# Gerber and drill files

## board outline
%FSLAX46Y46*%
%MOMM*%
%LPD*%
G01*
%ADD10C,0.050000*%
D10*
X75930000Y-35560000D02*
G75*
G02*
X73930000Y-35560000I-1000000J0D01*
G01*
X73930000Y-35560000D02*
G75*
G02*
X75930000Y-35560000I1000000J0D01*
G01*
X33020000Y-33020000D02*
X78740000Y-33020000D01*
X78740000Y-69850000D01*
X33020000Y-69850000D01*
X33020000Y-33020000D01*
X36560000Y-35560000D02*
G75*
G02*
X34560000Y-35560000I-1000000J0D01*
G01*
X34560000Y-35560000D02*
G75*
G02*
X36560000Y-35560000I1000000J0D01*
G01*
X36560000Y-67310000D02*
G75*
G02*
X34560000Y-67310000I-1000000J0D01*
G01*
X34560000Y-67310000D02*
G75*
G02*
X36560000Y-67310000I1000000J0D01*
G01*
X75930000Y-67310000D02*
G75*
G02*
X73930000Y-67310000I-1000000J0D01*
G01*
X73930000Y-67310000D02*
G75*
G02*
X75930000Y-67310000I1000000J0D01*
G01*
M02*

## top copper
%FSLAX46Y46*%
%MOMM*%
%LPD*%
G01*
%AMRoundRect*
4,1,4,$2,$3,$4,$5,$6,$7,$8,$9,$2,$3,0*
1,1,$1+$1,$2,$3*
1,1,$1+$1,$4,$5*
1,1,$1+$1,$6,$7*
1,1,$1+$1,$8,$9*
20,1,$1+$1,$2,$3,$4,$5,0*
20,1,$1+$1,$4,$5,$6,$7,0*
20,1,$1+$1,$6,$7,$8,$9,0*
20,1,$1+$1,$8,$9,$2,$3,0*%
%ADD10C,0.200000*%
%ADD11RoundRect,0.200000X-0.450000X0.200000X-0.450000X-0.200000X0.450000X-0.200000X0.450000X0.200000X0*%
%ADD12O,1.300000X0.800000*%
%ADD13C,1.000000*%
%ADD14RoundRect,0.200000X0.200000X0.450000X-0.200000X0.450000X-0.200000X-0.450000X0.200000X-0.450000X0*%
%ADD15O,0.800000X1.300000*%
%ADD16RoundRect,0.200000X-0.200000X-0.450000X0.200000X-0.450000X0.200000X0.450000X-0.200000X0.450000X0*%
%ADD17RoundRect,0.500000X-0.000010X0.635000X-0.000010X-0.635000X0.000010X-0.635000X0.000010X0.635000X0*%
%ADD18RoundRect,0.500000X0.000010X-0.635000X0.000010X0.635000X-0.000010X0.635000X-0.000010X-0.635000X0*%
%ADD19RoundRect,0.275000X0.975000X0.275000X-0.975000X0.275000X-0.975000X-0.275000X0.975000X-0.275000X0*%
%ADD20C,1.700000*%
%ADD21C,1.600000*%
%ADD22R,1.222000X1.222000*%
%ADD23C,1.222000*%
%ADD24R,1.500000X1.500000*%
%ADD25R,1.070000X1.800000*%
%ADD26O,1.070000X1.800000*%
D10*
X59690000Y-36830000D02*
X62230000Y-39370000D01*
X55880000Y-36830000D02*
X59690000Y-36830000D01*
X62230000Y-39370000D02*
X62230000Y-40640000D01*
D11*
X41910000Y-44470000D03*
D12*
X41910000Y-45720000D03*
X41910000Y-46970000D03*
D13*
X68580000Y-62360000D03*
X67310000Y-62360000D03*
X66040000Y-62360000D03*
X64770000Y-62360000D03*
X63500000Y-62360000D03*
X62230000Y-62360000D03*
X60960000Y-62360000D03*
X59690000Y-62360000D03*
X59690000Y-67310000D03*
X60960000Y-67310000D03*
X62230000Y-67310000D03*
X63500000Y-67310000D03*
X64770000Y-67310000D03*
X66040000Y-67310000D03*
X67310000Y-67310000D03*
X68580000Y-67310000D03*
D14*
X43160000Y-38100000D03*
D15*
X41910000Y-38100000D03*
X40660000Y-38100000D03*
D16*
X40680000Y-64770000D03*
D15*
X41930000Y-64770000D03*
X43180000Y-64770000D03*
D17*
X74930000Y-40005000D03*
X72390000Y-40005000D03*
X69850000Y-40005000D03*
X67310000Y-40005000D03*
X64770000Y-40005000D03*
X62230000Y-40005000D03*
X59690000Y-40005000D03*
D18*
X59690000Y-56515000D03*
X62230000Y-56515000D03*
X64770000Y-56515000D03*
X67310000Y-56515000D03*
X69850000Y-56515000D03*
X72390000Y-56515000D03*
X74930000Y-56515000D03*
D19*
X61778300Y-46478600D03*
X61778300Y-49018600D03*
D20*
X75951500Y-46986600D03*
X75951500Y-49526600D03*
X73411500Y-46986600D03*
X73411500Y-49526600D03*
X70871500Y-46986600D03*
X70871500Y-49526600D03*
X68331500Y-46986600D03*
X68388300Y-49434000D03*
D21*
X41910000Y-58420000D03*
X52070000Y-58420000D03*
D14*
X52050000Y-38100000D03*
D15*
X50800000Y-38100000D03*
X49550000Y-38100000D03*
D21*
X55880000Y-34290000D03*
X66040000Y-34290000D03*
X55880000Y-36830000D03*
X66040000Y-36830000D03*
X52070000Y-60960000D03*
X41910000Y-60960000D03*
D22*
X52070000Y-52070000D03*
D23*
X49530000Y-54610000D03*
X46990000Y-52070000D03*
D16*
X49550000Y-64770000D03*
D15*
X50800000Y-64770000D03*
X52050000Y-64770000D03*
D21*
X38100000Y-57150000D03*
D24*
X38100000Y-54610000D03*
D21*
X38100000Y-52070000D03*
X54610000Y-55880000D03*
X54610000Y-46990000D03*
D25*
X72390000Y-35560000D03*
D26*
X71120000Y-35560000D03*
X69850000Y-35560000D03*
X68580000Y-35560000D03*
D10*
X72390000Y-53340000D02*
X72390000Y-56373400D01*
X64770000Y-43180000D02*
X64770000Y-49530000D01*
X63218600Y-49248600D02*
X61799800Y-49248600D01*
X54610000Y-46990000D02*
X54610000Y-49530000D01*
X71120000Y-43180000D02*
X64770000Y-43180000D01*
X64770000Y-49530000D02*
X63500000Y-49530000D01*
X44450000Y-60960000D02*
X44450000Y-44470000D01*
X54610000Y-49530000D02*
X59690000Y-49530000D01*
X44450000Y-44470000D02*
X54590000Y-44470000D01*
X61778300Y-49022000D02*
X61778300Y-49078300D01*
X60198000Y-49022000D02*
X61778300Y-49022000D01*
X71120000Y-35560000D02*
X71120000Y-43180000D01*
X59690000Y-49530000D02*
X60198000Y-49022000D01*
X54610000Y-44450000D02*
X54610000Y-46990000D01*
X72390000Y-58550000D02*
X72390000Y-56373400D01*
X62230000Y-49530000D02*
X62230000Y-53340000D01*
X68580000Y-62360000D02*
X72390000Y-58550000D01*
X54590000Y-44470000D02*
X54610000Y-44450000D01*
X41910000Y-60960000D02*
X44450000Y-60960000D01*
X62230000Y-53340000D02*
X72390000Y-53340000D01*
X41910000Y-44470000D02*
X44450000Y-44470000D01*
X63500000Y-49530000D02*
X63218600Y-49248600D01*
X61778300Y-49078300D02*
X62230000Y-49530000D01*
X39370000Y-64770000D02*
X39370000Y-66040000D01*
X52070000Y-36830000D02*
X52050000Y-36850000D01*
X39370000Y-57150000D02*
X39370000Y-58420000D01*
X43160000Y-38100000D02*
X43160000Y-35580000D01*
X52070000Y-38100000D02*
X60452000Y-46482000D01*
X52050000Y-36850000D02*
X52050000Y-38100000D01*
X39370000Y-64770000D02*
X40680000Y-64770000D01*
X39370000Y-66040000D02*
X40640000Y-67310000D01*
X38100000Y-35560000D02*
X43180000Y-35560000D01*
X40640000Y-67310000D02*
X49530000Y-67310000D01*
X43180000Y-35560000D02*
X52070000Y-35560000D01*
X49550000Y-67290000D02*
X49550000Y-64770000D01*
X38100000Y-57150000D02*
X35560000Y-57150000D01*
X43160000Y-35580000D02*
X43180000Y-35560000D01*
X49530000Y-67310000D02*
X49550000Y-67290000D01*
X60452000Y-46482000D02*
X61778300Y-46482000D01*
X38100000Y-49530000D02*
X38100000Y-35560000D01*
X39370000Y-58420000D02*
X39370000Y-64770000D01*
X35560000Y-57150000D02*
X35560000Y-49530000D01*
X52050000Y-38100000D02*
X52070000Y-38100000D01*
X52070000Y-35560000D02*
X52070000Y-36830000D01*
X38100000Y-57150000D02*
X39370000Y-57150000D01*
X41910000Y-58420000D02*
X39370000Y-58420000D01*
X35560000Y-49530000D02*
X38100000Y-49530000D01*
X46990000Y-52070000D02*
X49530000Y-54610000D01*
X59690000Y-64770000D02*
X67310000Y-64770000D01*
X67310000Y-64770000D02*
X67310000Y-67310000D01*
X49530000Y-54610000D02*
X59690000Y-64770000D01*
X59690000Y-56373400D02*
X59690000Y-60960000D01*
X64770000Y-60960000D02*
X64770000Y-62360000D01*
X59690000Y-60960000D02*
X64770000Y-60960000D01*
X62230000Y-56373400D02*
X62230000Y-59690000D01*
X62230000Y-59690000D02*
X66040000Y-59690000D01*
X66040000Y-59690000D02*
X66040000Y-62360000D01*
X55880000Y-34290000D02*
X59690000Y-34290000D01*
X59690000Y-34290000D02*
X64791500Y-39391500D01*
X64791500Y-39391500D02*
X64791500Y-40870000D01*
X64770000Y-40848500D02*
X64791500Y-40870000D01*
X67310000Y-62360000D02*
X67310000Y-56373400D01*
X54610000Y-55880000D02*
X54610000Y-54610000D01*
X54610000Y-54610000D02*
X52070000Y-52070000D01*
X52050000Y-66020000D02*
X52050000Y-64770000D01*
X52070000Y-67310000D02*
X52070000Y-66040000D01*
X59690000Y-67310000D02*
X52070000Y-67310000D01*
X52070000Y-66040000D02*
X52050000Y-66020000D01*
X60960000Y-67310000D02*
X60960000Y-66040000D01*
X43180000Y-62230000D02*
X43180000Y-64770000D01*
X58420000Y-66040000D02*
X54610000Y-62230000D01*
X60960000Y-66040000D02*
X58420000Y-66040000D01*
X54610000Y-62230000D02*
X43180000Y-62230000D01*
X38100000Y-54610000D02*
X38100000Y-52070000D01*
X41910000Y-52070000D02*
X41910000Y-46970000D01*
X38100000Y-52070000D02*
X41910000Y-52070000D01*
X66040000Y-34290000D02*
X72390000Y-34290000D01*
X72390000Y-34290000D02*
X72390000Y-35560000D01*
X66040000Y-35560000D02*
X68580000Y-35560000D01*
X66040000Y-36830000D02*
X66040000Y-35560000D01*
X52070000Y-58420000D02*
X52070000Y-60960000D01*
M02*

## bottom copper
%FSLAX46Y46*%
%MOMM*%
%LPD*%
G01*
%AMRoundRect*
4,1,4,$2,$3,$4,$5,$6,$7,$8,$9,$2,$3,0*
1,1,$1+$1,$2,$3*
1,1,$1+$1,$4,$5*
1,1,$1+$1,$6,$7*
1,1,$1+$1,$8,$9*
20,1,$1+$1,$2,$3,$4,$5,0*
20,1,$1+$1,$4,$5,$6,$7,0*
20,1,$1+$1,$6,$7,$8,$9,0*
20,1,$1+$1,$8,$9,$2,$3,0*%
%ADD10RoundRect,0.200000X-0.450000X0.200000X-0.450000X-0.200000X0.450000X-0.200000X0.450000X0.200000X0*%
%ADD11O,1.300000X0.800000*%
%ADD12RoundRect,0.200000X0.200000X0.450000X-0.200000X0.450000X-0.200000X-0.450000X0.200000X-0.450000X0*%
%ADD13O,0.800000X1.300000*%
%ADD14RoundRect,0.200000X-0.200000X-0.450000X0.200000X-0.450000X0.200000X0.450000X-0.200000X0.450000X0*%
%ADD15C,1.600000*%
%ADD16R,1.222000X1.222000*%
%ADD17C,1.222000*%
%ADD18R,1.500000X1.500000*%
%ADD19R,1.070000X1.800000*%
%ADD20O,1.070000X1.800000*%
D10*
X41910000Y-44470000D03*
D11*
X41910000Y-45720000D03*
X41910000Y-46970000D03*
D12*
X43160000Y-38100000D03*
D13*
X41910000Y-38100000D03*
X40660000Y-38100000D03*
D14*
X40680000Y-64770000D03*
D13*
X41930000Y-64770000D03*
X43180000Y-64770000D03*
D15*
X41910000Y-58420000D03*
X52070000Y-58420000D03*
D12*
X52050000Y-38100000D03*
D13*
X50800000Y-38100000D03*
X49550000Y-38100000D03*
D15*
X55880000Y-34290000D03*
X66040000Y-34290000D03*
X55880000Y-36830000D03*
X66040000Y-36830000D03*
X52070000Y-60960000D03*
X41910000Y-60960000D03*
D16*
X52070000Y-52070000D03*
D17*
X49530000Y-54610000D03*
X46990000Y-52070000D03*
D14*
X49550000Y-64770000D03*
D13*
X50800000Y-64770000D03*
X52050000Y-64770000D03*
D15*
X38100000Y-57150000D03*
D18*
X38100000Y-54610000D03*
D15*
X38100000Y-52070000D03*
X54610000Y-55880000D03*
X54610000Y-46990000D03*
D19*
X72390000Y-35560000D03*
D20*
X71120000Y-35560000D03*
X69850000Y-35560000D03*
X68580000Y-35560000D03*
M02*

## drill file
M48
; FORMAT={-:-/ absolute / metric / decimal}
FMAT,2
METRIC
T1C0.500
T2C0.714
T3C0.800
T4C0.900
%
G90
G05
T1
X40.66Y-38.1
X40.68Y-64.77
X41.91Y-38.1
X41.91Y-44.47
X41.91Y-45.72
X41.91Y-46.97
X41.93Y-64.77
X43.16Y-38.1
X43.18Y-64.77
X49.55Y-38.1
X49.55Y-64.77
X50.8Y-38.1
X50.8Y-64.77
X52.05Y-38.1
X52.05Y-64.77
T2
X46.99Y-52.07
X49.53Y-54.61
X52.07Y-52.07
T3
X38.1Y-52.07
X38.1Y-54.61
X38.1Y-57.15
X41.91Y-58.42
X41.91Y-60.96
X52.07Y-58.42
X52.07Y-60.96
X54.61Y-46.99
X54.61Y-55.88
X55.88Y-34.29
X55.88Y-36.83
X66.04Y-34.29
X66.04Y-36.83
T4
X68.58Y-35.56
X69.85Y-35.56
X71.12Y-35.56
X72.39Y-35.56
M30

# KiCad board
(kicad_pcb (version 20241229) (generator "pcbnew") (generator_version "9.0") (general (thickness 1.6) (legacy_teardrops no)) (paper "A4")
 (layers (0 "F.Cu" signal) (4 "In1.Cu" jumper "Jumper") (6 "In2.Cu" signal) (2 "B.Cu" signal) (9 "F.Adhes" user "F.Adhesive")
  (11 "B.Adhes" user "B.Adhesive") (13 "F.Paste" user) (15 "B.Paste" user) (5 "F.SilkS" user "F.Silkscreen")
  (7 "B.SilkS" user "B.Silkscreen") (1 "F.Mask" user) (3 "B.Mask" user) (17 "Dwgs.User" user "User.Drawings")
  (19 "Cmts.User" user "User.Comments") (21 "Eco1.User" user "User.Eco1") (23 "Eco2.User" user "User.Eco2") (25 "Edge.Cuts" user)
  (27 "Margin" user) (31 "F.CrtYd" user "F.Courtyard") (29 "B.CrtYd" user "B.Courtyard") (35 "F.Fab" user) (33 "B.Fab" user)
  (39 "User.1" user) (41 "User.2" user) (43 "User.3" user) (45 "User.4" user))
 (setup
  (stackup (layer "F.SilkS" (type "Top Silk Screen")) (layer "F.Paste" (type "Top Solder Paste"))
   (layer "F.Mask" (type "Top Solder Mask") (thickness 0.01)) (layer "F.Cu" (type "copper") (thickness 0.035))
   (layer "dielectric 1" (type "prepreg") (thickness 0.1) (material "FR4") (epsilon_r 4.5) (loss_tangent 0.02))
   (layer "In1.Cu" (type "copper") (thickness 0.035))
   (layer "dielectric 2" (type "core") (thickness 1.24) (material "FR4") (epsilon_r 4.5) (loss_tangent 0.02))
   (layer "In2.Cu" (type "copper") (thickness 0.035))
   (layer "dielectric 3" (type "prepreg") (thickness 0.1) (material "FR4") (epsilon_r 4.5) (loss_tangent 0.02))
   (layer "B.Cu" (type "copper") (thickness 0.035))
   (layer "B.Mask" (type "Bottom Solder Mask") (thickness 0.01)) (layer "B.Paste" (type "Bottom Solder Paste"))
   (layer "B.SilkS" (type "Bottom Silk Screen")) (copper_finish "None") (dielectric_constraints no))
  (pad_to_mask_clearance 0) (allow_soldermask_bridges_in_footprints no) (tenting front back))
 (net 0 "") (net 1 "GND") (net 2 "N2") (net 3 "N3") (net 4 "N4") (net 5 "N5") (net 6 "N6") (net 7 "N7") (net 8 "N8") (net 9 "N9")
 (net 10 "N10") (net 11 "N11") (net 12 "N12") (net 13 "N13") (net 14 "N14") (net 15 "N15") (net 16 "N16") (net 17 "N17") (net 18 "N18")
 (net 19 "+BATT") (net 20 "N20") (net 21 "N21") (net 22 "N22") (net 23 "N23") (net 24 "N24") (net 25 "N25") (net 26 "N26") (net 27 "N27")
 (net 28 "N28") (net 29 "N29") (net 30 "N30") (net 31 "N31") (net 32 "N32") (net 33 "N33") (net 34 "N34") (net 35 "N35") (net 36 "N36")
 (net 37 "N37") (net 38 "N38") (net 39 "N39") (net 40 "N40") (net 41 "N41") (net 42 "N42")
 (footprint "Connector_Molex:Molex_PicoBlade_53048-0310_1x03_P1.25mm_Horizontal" (layer "F.Cu") (at 41.91 44.47 -90)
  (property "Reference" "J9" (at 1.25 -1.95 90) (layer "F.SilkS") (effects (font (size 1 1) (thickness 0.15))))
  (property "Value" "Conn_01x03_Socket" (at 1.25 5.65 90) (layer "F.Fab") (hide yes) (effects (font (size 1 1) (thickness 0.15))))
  (pad "1" thru_hole roundrect (at 0 0 270) (size 0.8 1.3) (drill 0.5) (layers "*.Cu" "*.Mask") (remove_unused_layers no)
   (roundrect_rratio 0.25) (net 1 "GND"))
  (pad "2" thru_hole oval (at 1.25 0 270) (size 0.8 1.3) (drill 0.5) (layers "*.Cu" "*.Mask") (remove_unused_layers no) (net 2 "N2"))
  (pad "3" thru_hole oval (at 2.5 0 270) (size 0.8 1.3) (drill 0.5) (layers "*.Cu" "*.Mask") (remove_unused_layers no) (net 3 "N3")))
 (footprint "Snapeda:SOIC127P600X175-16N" (layer "F.Cu") (at 63.5 64.835 -90)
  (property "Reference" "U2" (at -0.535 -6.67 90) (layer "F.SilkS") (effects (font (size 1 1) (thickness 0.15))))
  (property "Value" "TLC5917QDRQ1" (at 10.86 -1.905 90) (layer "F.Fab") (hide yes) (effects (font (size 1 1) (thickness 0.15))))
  (pad "1" smd circle (at -2.475 -5.08 270) (size 1 1) (layers "F.Cu" "F.Mask" "F.Paste") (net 1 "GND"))
  (pad "2" smd circle (at -2.475 -3.81 270) (size 1 1) (layers "F.Cu" "F.Mask" "F.Paste") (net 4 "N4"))
  (pad "3" smd circle (at -2.475 -2.54 270) (size 1 1) (layers "F.Cu" "F.Mask" "F.Paste") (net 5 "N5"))
  (pad "4" smd circle (at -2.475 -1.27 270) (size 1 1) (layers "F.Cu" "F.Mask" "F.Paste") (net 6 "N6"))
  (pad "5" smd circle (at -2.475 0 270) (size 1 1) (layers "F.Cu" "F.Mask" "F.Paste") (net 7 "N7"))
  (pad "6" smd circle (at -2.475 1.27 270) (size 1 1) (layers "F.Cu" "F.Mask" "F.Paste") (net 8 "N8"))
  (pad "7" smd circle (at -2.475 2.54 270) (size 1 1) (layers "F.Cu" "F.Mask" "F.Paste") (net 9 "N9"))
  (pad "8" smd circle (at -2.475 3.81 270) (size 1 1) (layers "F.Cu" "F.Mask" "F.Paste") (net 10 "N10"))
  (pad "9" smd circle (at 2.475 3.81 270) (size 1 1) (layers "F.Cu" "F.Mask" "F.Paste") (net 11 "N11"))
  (pad "10" smd circle (at 2.475 2.54 270) (size 1 1) (layers "F.Cu" "F.Mask" "F.Paste") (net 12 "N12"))
  (pad "11" smd circle (at 2.475 1.27 270) (size 1 1) (layers "F.Cu" "F.Mask" "F.Paste") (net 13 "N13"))
  (pad "12" smd circle (at 2.475 0 270) (size 1 1) (layers "F.Cu" "F.Mask" "F.Paste") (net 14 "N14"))
  (pad "13" smd circle (at 2.475 -1.27 270) (size 1 1) (layers "F.Cu" "F.Mask" "F.Paste") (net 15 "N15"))
  (pad "14" smd circle (at 2.475 -2.54 270) (size 1 1) (layers "F.Cu" "F.Mask" "F.Paste") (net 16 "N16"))
  (pad "15" smd circle (at 2.475 -3.81 270) (size 1 1) (layers "F.Cu" "F.Mask" "F.Paste") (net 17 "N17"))
  (pad "16" smd circle (at 2.475 -5.08 270) (size 1 1) (layers "F.Cu" "F.Mask" "F.Paste") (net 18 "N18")))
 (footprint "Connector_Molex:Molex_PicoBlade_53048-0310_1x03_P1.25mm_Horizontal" (layer "F.Cu") (at 43.16 38.1 180)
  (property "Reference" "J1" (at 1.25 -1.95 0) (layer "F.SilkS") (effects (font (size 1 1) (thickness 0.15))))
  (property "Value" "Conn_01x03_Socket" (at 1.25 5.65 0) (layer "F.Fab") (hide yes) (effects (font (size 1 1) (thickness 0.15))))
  (pad "1" thru_hole roundrect (at 0 0 180) (size 0.8 1.3) (drill 0.5) (layers "*.Cu" "*.Mask") (remove_unused_layers no)
   (roundrect_rratio 0.25) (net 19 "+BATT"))
  (pad "2" thru_hole oval (at 1.25 0 180) (size 0.8 1.3) (drill 0.5) (layers "*.Cu" "*.Mask") (remove_unused_layers no) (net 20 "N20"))
  (pad "3" thru_hole oval (at 2.5 0 180) (size 0.8 1.3) (drill 0.5) (layers "*.Cu" "*.Mask") (remove_unused_layers no) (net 13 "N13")))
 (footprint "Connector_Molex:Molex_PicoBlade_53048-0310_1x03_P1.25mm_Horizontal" (layer "F.Cu") (at 40.68 64.77)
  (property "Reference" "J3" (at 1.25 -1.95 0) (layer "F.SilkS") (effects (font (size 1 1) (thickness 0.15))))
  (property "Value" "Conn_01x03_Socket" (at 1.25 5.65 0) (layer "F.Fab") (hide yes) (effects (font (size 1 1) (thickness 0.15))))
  (pad "1" thru_hole roundrect (at 0 0) (size 0.8 1.3) (drill 0.5) (layers "*.Cu" "*.Mask") (remove_unused_layers no)
   (roundrect_rratio 0.25) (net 19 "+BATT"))
  (pad "2" thru_hole oval (at 1.25 0) (size 0.8 1.3) (drill 0.5) (layers "*.Cu" "*.Mask") (remove_unused_layers no) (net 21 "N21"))
  (pad "3" thru_hole oval (at 2.5 0) (size 0.8 1.3) (drill 0.5) (layers "*.Cu" "*.Mask") (remove_unused_layers no) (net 12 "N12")))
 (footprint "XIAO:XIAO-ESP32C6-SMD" (layer "F.Cu") (at 67.31 48.26 -90)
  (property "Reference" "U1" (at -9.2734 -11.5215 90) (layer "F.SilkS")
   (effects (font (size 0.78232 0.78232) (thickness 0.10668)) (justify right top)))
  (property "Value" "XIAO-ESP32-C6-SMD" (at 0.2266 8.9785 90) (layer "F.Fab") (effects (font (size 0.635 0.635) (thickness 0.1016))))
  (pad "1" smd roundrect (at -7.62 -7.62 270) (size 2.27 1) (drill (offset -0.635 0)) (layers "F.Cu" "F.Mask" "F.Paste")
   (roundrect_rratio 0.5) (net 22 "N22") (solder_mask_margin 0.0508) (thermal_bridge_angle 45))
  (pad "2" smd roundrect (at -7.62 -5.08 270) (size 2.27 1) (drill (offset -0.635 0)) (layers "F.Cu" "F.Mask" "F.Paste")
   (roundrect_rratio 0.5) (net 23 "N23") (solder_mask_margin 0.0508) (thermal_bridge_angle 45))
  (pad "3" smd roundrect (at -7.62 -2.54 270) (size 2.27 1) (drill (offset -0.635 0)) (layers "F.Cu" "F.Mask" "F.Paste")
   (roundrect_rratio 0.5) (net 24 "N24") (solder_mask_margin 0.0508) (thermal_bridge_angle 45))
  (pad "4" smd roundrect (at -7.62 0 270) (size 2.27 1) (drill (offset -0.635 0)) (layers "F.Cu" "F.Mask" "F.Paste") (roundrect_rratio 0.5)
   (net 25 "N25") (solder_mask_margin 0.0508) (thermal_bridge_angle 45))
  (pad "5" smd roundrect (at -7.62 2.54 270) (size 2.27 1) (drill (offset -0.635 0)) (layers "F.Cu" "F.Mask" "F.Paste")
   (roundrect_rratio 0.5) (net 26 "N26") (solder_mask_margin 0.0508) (thermal_bridge_angle 45))
  (pad "6" smd roundrect (at -7.62 5.08 270) (size 2.27 1) (drill (offset -0.635 0)) (layers "F.Cu" "F.Mask" "F.Paste")
   (roundrect_rratio 0.5) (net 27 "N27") (solder_mask_margin 0.0508) (thermal_bridge_angle 45))
  (pad "7" smd roundrect (at -7.62 7.62 270) (size 2.27 1) (drill (offset -0.635 0)) (layers "F.Cu" "F.Mask" "F.Paste")
   (roundrect_rratio 0.5) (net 15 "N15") (solder_mask_margin 0.0508) (thermal_bridge_angle 45))
  (pad "8" smd roundrect (at 7.62 7.62 90) (size 2.27 1) (drill (offset -0.635 0)) (layers "F.Cu" "F.Mask" "F.Paste") (roundrect_rratio 0.5)
   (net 6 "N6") (solder_mask_margin 0.0508) (thermal_bridge_angle 45))
  (pad "9" smd roundrect (at 7.62 5.08 90) (size 2.27 1) (drill (offset -0.635 0)) (layers "F.Cu" "F.Mask" "F.Paste") (roundrect_rratio 0.5)
   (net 5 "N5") (solder_mask_margin 0.0508) (thermal_bridge_angle 45))
  (pad "10" smd roundrect (at 7.62 2.54 90) (size 2.27 1) (drill (offset -0.635 0)) (layers "F.Cu" "F.Mask" "F.Paste")
   (roundrect_rratio 0.5) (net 16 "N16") (solder_mask_margin 0.0508) (thermal_bridge_angle 45))
  (pad "11" smd roundrect (at 7.62 0 90) (size 2.27 1) (drill (offset -0.635 0)) (layers "F.Cu" "F.Mask" "F.Paste") (roundrect_rratio 0.5)
   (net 4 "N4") (solder_mask_margin 0.0508) (thermal_bridge_angle 45))
  (pad "12" smd roundrect (at 7.62 -2.54 90) (size 2.27 1) (drill (offset -0.635 0)) (layers "F.Cu" "F.Mask" "F.Paste")
   (roundrect_rratio 0.5) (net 18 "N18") (solder_mask_margin 0.0508) (thermal_bridge_angle 45))
  (pad "13" smd roundrect (at 7.62 -5.08 90) (size 2.27 1) (drill (offset -0.635 0)) (layers "F.Cu" "F.Mask" "F.Paste")
   (roundrect_rratio 0.5) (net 1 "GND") (solder_mask_margin 0.0508) (thermal_bridge_angle 45))
  (pad "14" smd roundrect (at 7.62 -7.62 90) (size 2.27 1) (drill (offset -0.635 0)) (layers "F.Cu" "F.Mask" "F.Paste")
   (roundrect_rratio 0.5) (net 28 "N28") (solder_mask_margin 0.0508) (thermal_bridge_angle 45))
  (pad "15" smd roundrect (at -1.7814 5.5317 180) (size 2.5 1.1) (layers "F.Cu" "F.Mask" "F.Paste") (roundrect_rratio 0.25) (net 19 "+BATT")
   (solder_mask_margin 0.0508) (thermal_bridge_angle 45))
  (pad "16" smd roundrect (at 0.7586 5.5317 180) (size 2.5 1.1) (layers "F.Cu" "F.Mask" "F.Paste") (roundrect_rratio 0.25) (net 1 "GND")
   (solder_mask_margin 0.0508) (thermal_bridge_angle 45))
  (pad "17" smd circle (at -1.2734 -8.6415 270) (size 1.7 1.7) (layers "F.Cu" "F.Mask" "F.Paste") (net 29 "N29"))
  (pad "18" smd circle (at 1.2666 -8.6415 270) (size 1.7 1.7) (layers "F.Cu" "F.Mask" "F.Paste") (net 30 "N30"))
  (pad "19" smd circle (at -1.2734 -6.1015 270) (size 1.7 1.7) (layers "F.Cu" "F.Mask" "F.Paste") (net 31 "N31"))
  (pad "20" smd circle (at 1.2666 -6.1015 270) (size 1.7 1.7) (layers "F.Cu" "F.Mask" "F.Paste") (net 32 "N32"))
  (pad "21" smd circle (at -1.2734 -3.5615 270) (size 1.7 1.7) (layers "F.Cu" "F.Mask" "F.Paste") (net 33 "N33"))
  (pad "22" smd circle (at 1.2666 -3.5615 270) (size 1.7 1.7) (layers "F.Cu" "F.Mask" "F.Paste") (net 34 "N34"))
  (pad "23" smd circle (at -1.2734 -1.0215 270) (size 1.7 1.7) (layers "F.Cu" "F.Mask" "F.Paste") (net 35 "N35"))
  (pad "24" smd circle (at 1.174 -1.0783 270) (size 1.7 1.7) (layers "F.Cu" "F.Mask" "F.Paste") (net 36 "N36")))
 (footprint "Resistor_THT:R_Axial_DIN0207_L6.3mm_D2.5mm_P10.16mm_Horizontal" (layer "F.Cu") (at 41.91 58.42)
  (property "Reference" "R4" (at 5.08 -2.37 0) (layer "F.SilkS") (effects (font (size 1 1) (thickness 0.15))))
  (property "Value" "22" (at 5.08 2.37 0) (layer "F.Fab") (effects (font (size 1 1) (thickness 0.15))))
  (pad "1" thru_hole circle (at 0 0) (size 1.6 1.6) (drill 0.8) (layers "*.Cu" "*.Mask") (remove_unused_layers no) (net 19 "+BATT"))
  (pad "2" thru_hole circle (at 10.16 0) (size 1.6 1.6) (drill 0.8) (layers "*.Cu" "*.Mask") (remove_unused_layers no) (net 22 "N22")))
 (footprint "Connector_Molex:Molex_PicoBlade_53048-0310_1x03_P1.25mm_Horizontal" (layer "F.Cu") (at 52.05 38.1 180)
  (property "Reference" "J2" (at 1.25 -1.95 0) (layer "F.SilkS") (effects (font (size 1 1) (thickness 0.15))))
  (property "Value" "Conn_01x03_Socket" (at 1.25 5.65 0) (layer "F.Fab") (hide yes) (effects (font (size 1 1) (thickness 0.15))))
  (pad "1" thru_hole roundrect (at 0 0 180) (size 0.8 1.3) (drill 0.5) (layers "*.Cu" "*.Mask") (remove_unused_layers no)
   (roundrect_rratio 0.25) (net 19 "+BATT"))
  (pad "2" thru_hole oval (at 1.25 0 180) (size 0.8 1.3) (drill 0.5) (layers "*.Cu" "*.Mask") (remove_unused_layers no) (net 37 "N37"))
  (pad "3" thru_hole oval (at 2.5 0 180) (size 0.8 1.3) (drill 0.5) (layers "*.Cu" "*.Mask") (remove_unused_layers no) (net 14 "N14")))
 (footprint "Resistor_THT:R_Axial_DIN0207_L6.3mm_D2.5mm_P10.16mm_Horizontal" (layer "F.Cu") (at 55.88 34.29)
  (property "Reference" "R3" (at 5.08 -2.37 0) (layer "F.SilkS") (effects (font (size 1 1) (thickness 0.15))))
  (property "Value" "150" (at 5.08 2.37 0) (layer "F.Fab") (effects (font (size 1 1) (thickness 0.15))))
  (pad "1" thru_hole circle (at 0 0) (size 1.6 1.6) (drill 0.8) (layers "*.Cu" "*.Mask") (remove_unused_layers no) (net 26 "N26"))
  (pad "2" thru_hole circle (at 10.16 0) (size 1.6 1.6) (drill 0.8) (layers "*.Cu" "*.Mask") (remove_unused_layers no) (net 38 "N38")))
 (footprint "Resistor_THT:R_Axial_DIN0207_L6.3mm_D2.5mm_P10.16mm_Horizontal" (layer "F.Cu") (at 55.88 36.83)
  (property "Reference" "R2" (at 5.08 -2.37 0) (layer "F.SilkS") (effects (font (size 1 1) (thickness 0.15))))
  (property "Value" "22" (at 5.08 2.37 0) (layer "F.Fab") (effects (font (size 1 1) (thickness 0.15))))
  (pad "1" thru_hole circle (at 0 0) (size 1.6 1.6) (drill 0.8) (layers "*.Cu" "*.Mask") (remove_unused_layers no) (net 27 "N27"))
  (pad "2" thru_hole circle (at 10.16 0) (size 1.6 1.6) (drill 0.8) (layers "*.Cu" "*.Mask") (remove_unused_layers no) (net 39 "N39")))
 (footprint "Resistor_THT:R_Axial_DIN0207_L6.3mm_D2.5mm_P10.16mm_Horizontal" (layer "F.Cu") (at 52.07 60.96 180)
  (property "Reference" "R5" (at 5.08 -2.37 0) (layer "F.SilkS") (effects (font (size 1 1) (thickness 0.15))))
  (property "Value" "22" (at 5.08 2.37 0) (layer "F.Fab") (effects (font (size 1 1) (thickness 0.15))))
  (pad "1" thru_hole circle (at 0 0 180) (size 1.6 1.6) (drill 0.8) (layers "*.Cu" "*.Mask") (remove_unused_layers no) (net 22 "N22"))
  (pad "2" thru_hole circle (at 10.16 0 180) (size 1.6 1.6) (drill 0.8) (layers "*.Cu" "*.Mask") (remove_unused_layers no) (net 1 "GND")))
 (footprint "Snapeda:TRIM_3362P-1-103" (layer "F.Cu") (at 49.53 52.07 180)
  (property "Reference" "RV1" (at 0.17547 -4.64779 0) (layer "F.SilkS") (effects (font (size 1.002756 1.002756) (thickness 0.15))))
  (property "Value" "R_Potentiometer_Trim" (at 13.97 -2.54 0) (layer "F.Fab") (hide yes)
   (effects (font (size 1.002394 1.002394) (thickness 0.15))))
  (pad "1" thru_hole rect (at -2.54 0 180) (size 1.222 1.222) (drill 0.714) (layers "*.Cu" "*.Mask") (remove_unused_layers no)
   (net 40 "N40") (solder_mask_margin 0.102))
  (pad "2" thru_hole circle (at 0 -2.54 180) (size 1.222 1.222) (drill 0.714) (layers "*.Cu" "*.Mask") (remove_unused_layers no)
   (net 17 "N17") (solder_mask_margin 0.102))
  (pad "3" thru_hole circle (at 2.54 0 180) (size 1.222 1.222) (drill 0.714) (layers "*.Cu" "*.Mask") (remove_unused_layers no)
   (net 17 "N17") (solder_mask_margin 0.102)))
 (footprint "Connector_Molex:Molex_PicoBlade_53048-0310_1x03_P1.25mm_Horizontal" (layer "F.Cu") (at 49.55 64.77)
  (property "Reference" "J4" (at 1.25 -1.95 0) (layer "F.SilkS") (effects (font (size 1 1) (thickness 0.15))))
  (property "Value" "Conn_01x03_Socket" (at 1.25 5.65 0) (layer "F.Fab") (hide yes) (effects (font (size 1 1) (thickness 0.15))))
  (pad "1" thru_hole roundrect (at 0 0) (size 0.8 1.3) (drill 0.5) (layers "*.Cu" "*.Mask") (remove_unused_layers no)
   (roundrect_rratio 0.25) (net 19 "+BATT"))
  (pad "2" thru_hole oval (at 1.25 0) (size 0.8 1.3) (drill 0.5) (layers "*.Cu" "*.Mask") (remove_unused_layers no) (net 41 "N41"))
  (pad "3" thru_hole oval (at 2.5 0) (size 0.8 1.3) (drill 0.5) (layers "*.Cu" "*.Mask") (remove_unused_layers no) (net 11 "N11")))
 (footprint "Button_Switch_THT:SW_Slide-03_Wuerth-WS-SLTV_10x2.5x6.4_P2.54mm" (layer "F.Cu") (at 38.1 54.61 90)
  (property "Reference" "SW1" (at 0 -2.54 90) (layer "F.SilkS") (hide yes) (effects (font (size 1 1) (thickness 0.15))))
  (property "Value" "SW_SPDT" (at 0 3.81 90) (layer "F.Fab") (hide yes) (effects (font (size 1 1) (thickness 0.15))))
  (pad "1" thru_hole circle (at -2.54 0 90) (size 1.6 1.6) (drill 0.8) (layers "*.Cu" "*.Mask") (remove_unused_layers no) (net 19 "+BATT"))
  (pad "2" thru_hole rect (at 0 0 90) (size 1.5 1.5) (drill 0.8) (layers "*.Cu" "*.Mask") (remove_unused_layers no) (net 3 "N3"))
  (pad "3" thru_hole circle (at 2.54 0 90) (size 1.6 1.6) (drill 0.8) (layers "*.Cu" "*.Mask") (remove_unused_layers no) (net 3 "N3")))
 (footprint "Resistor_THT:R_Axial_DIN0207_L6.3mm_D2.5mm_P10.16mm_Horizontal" (layer "F.Cu") (at 54.61 55.88 90)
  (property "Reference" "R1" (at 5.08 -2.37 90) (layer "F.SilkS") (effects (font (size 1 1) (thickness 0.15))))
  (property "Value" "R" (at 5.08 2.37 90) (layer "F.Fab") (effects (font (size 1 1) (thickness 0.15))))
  (pad "1" thru_hole circle (at 0 0 90) (size 1.6 1.6) (drill 0.8) (layers "*.Cu" "*.Mask") (remove_unused_layers no) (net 40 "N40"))
  (pad "2" thru_hole circle (at 8.89 0 90) (size 1.6 1.6) (drill 0.8) (layers "*.Cu" "*.Mask") (remove_unused_layers no) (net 1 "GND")))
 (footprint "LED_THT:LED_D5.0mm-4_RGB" (layer "F.Cu") (at 72.39 35.56 180)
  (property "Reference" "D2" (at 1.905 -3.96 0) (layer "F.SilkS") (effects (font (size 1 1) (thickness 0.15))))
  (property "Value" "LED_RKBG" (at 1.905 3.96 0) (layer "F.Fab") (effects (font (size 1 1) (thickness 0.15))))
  (pad "1" thru_hole rect (at 0 0 180) (size 1.07 1.8) (drill 0.9) (layers "*.Cu" "*.Mask") (remove_unused_layers no) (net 38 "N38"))
  (pad "2" thru_hole oval (at 1.27 0 180) (size 1.07 1.8) (drill 0.9) (layers "*.Cu" "*.Mask") (remove_unused_layers no) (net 1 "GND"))
  (pad "3" thru_hole oval (at 2.54 0 180) (size 1.07 1.8) (drill 0.9) (layers "*.Cu" "*.Mask") (remove_unused_layers no) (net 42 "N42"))
  (pad "4" thru_hole oval (at 3.81 0 180) (size 1.07 1.8) (drill 0.9) (layers "*.Cu" "*.Mask") (remove_unused_layers no) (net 39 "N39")))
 (gr_line (start 59.69 36.83) (end 62.23 39.37) (stroke (width 0.2) (type default)) (layer "F.Cu") (net 27))
 (gr_line (start 55.88 36.83) (end 59.69 36.83) (stroke (width 0.2) (type default)) (layer "F.Cu") (net 27))
 (gr_line (start 62.23 39.37) (end 62.23 40.64) (stroke (width 0.2) (type default)) (layer "F.Cu") (net 27))
 (gr_circle (center 74.93 35.56) (end 73.93 35.56) (stroke (width 0.05) (type default)) (fill no) (layer "Edge.Cuts"))
 (gr_rect (start 33.02 33.02) (end 78.74 69.85) (stroke (width 0.05) (type default)) (fill no) (layer "Edge.Cuts"))
 (gr_circle (center 35.56 35.56) (end 34.56 35.56) (stroke (width 0.05) (type default)) (fill no) (layer "Edge.Cuts"))
 (gr_circle (center 35.56 67.31) (end 34.56 67.31) (stroke (width 0.05) (type default)) (fill no) (layer "Edge.Cuts"))
 (gr_circle (center 74.93 67.31) (end 73.93 67.31) (stroke (width 0.05) (type default)) (fill no) (layer "Edge.Cuts"))
 (segment (start 72.39 53.34) (end 72.39 56.3734) (width 0.2) (layer "F.Cu") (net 1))
 (segment (start 64.77 43.18) (end 64.77 49.53) (width 0.2) (layer "F.Cu") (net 1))
 (segment (start 63.2186 49.2486) (end 61.7998 49.2486) (width 0.2) (layer "F.Cu") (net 1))
 (segment (start 54.61 46.99) (end 54.61 49.53) (width 0.2) (layer "F.Cu") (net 1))
 (segment (start 71.12 43.18) (end 64.77 43.18) (width 0.2) (layer "F.Cu") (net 1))
 (segment (start 64.77 49.53) (end 63.5 49.53) (width 0.2) (layer "F.Cu") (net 1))
 (segment (start 44.45 60.96) (end 44.45 44.47) (width 0.2) (layer "F.Cu") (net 1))
 (segment (start 54.61 49.53) (end 59.69 49.53) (width 0.2) (layer "F.Cu") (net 1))
 (segment (start 44.45 44.47) (end 54.59 44.47) (width 0.2) (layer "F.Cu") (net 1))
 (segment (start 61.7783 49.022) (end 61.7783 49.0783) (width 0.2) (layer "F.Cu") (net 1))
 (segment (start 60.198 49.022) (end 61.7783 49.022) (width 0.2) (layer "F.Cu") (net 1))
 (segment (start 71.12 35.56) (end 71.12 43.18) (width 0.2) (layer "F.Cu") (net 1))
 (segment (start 59.69 49.53) (end 60.198 49.022) (width 0.2) (layer "F.Cu") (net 1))
 (segment (start 54.61 44.45) (end 54.61 46.99) (width 0.2) (layer "F.Cu") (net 1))
 (segment (start 72.39 58.55) (end 72.39 56.3734) (width 0.2) (layer "F.Cu") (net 1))
 (segment (start 62.23 49.53) (end 62.23 53.34) (width 0.2) (layer "F.Cu") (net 1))
 (segment (start 68.58 62.36) (end 72.39 58.55) (width 0.2) (layer "F.Cu") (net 1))
 (segment (start 54.59 44.47) (end 54.61 44.45) (width 0.2) (layer "F.Cu") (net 1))
 (segment (start 41.91 60.96) (end 44.45 60.96) (width 0.2) (layer "F.Cu") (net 1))
 (segment (start 62.23 53.34) (end 72.39 53.34) (width 0.2) (layer "F.Cu") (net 1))
 (segment (start 41.91 44.47) (end 44.45 44.47) (width 0.2) (layer "F.Cu") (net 1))
 (segment (start 63.5 49.53) (end 63.2186 49.2486) (width 0.2) (layer "F.Cu") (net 1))
 (segment (start 61.7783 49.0783) (end 62.23 49.53) (width 0.2) (layer "F.Cu") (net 1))
 (segment (start 39.37 64.77) (end 39.37 66.04) (width 0.2) (layer "F.Cu") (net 19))
 (segment (start 52.07 36.83) (end 52.05 36.85) (width 0.2) (layer "F.Cu") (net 19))
 (segment (start 39.37 57.15) (end 39.37 58.42) (width 0.2) (layer "F.Cu") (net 19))
 (segment (start 43.16 38.1) (end 43.16 35.58) (width 0.2) (layer "F.Cu") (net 19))
 (segment (start 52.07 38.1) (end 60.452 46.482) (width 0.2) (layer "F.Cu") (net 19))
 (segment (start 52.05 36.85) (end 52.05 38.1) (width 0.2) (layer "F.Cu") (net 19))
 (segment (start 39.37 64.77) (end 40.68 64.77) (width 0.2) (layer "F.Cu") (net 19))
 (segment (start 39.37 66.04) (end 40.64 67.31) (width 0.2) (layer "F.Cu") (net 19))
 (segment (start 38.1 35.56) (end 43.18 35.56) (width 0.2) (layer "F.Cu") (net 19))
 (segment (start 40.64 67.31) (end 49.53 67.31) (width 0.2) (layer "F.Cu") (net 19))
 (segment (start 43.18 35.56) (end 52.07 35.56) (width 0.2) (layer "F.Cu") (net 19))
 (segment (start 49.55 67.29) (end 49.55 64.77) (width 0.2) (layer "F.Cu") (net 19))
 (segment (start 38.1 57.15) (end 35.56 57.15) (width 0.2) (layer "F.Cu") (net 19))
 (segment (start 43.16 35.58) (end 43.18 35.56) (width 0.2) (layer "F.Cu") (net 19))
 (segment (start 49.53 67.31) (end 49.55 67.29) (width 0.2) (layer "F.Cu") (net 19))
 (segment (start 60.452 46.482) (end 61.7783 46.482) (width 0.2) (layer "F.Cu") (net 19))
 (segment (start 38.1 49.53) (end 38.1 35.56) (width 0.2) (layer "F.Cu") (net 19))
 (segment (start 39.37 58.42) (end 39.37 64.77) (width 0.2) (layer "F.Cu") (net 19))
 (segment (start 35.56 57.15) (end 35.56 49.53) (width 0.2) (layer "F.Cu") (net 19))
 (segment (start 52.05 38.1) (end 52.07 38.1) (width 0.2) (layer "F.Cu") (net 19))
 (segment (start 52.07 35.56) (end 52.07 36.83) (width 0.2) (layer "F.Cu") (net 19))
 (segment (start 38.1 57.15) (end 39.37 57.15) (width 0.2) (layer "F.Cu") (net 19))
 (segment (start 41.91 58.42) (end 39.37 58.42) (width 0.2) (layer "F.Cu") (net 19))
 (segment (start 35.56 49.53) (end 38.1 49.53) (width 0.2) (layer "F.Cu") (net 19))
 (segment (start 46.99 52.07) (end 49.53 54.61) (width 0.2) (layer "F.Cu") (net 17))
 (segment (start 59.69 64.77) (end 67.31 64.77) (width 0.2) (layer "F.Cu") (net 17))
 (segment (start 67.31 64.77) (end 67.31 67.31) (width 0.2) (layer "F.Cu") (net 17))
 (segment (start 49.53 54.61) (end 59.69 64.77) (width 0.2) (layer "F.Cu") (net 17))
 (segment (start 59.69 56.3734) (end 59.69 60.96) (width 0.2) (layer "F.Cu") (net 6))
 (segment (start 64.77 60.96) (end 64.77 62.36) (width 0.2) (layer "F.Cu") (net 6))
 (segment (start 59.69 60.96) (end 64.77 60.96) (width 0.2) (layer "F.Cu") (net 6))
 (segment (start 62.23 56.3734) (end 62.23 59.69) (width 0.2) (layer "F.Cu") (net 5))
 (segment (start 62.23 59.69) (end 66.04 59.69) (width 0.2) (layer "F.Cu") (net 5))
 (segment (start 66.04 59.69) (end 66.04 62.36) (width 0.2) (layer "F.Cu") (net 5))
 (segment (start 55.88 34.29) (end 59.69 34.29) (width 0.2) (layer "F.Cu") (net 26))
 (segment (start 59.69 34.29) (end 64.7915 39.3915) (width 0.2) (layer "F.Cu") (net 26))
 (segment (start 64.7915 39.3915) (end 64.7915 40.87) (width 0.2) (layer "F.Cu") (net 26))
 (segment (start 64.77 40.8485) (end 64.7915 40.87) (width 0.2) (layer "F.Cu") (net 26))
 (segment (start 67.31 62.36) (end 67.31 56.3734) (width 0.2) (layer "F.Cu") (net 4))
 (segment (start 54.61 55.88) (end 54.61 54.61) (width 0.2) (layer "F.Cu") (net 40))
 (segment (start 54.61 54.61) (end 52.07 52.07) (width 0.2) (layer "F.Cu") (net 40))
 (segment (start 52.05 66.02) (end 52.05 64.77) (width 0.2) (layer "F.Cu") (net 11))
 (segment (start 52.07 67.31) (end 52.07 66.04) (width 0.2) (layer "F.Cu") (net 11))
 (segment (start 59.69 67.31) (end 52.07 67.31) (width 0.2) (layer "F.Cu") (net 11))
 (segment (start 52.07 66.04) (end 52.05 66.02) (width 0.2) (layer "F.Cu") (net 11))
 (segment (start 60.96 67.31) (end 60.96 66.04) (width 0.2) (layer "F.Cu") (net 12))
 (segment (start 43.18 62.23) (end 43.18 64.77) (width 0.2) (layer "F.Cu") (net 12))
 (segment (start 58.42 66.04) (end 54.61 62.23) (width 0.2) (layer "F.Cu") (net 12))
 (segment (start 60.96 66.04) (end 58.42 66.04) (width 0.2) (layer "F.Cu") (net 12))
 (segment (start 54.61 62.23) (end 43.18 62.23) (width 0.2) (layer "F.Cu") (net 12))
 (segment (start 38.1 54.61) (end 38.1 52.07) (width 0.2) (layer "F.Cu") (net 3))
 (segment (start 41.91 52.07) (end 41.91 46.97) (width 0.2) (layer "F.Cu") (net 3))
 (segment (start 38.1 52.07) (end 41.91 52.07) (width 0.2) (layer "F.Cu") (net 3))
 (segment (start 66.04 34.29) (end 72.39 34.29) (width 0.2) (layer "F.Cu") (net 38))
 (segment (start 72.39 34.29) (end 72.39 35.56) (width 0.2) (layer "F.Cu") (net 38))
 (segment (start 66.04 35.56) (end 68.58 35.56) (width 0.2) (layer "F.Cu") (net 39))
 (segment (start 66.04 36.83) (end 66.04 35.56) (width 0.2) (layer "F.Cu") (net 39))
 (segment (start 52.07 58.42) (end 52.07 60.96) (width 0.2) (layer "F.Cu") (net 22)))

